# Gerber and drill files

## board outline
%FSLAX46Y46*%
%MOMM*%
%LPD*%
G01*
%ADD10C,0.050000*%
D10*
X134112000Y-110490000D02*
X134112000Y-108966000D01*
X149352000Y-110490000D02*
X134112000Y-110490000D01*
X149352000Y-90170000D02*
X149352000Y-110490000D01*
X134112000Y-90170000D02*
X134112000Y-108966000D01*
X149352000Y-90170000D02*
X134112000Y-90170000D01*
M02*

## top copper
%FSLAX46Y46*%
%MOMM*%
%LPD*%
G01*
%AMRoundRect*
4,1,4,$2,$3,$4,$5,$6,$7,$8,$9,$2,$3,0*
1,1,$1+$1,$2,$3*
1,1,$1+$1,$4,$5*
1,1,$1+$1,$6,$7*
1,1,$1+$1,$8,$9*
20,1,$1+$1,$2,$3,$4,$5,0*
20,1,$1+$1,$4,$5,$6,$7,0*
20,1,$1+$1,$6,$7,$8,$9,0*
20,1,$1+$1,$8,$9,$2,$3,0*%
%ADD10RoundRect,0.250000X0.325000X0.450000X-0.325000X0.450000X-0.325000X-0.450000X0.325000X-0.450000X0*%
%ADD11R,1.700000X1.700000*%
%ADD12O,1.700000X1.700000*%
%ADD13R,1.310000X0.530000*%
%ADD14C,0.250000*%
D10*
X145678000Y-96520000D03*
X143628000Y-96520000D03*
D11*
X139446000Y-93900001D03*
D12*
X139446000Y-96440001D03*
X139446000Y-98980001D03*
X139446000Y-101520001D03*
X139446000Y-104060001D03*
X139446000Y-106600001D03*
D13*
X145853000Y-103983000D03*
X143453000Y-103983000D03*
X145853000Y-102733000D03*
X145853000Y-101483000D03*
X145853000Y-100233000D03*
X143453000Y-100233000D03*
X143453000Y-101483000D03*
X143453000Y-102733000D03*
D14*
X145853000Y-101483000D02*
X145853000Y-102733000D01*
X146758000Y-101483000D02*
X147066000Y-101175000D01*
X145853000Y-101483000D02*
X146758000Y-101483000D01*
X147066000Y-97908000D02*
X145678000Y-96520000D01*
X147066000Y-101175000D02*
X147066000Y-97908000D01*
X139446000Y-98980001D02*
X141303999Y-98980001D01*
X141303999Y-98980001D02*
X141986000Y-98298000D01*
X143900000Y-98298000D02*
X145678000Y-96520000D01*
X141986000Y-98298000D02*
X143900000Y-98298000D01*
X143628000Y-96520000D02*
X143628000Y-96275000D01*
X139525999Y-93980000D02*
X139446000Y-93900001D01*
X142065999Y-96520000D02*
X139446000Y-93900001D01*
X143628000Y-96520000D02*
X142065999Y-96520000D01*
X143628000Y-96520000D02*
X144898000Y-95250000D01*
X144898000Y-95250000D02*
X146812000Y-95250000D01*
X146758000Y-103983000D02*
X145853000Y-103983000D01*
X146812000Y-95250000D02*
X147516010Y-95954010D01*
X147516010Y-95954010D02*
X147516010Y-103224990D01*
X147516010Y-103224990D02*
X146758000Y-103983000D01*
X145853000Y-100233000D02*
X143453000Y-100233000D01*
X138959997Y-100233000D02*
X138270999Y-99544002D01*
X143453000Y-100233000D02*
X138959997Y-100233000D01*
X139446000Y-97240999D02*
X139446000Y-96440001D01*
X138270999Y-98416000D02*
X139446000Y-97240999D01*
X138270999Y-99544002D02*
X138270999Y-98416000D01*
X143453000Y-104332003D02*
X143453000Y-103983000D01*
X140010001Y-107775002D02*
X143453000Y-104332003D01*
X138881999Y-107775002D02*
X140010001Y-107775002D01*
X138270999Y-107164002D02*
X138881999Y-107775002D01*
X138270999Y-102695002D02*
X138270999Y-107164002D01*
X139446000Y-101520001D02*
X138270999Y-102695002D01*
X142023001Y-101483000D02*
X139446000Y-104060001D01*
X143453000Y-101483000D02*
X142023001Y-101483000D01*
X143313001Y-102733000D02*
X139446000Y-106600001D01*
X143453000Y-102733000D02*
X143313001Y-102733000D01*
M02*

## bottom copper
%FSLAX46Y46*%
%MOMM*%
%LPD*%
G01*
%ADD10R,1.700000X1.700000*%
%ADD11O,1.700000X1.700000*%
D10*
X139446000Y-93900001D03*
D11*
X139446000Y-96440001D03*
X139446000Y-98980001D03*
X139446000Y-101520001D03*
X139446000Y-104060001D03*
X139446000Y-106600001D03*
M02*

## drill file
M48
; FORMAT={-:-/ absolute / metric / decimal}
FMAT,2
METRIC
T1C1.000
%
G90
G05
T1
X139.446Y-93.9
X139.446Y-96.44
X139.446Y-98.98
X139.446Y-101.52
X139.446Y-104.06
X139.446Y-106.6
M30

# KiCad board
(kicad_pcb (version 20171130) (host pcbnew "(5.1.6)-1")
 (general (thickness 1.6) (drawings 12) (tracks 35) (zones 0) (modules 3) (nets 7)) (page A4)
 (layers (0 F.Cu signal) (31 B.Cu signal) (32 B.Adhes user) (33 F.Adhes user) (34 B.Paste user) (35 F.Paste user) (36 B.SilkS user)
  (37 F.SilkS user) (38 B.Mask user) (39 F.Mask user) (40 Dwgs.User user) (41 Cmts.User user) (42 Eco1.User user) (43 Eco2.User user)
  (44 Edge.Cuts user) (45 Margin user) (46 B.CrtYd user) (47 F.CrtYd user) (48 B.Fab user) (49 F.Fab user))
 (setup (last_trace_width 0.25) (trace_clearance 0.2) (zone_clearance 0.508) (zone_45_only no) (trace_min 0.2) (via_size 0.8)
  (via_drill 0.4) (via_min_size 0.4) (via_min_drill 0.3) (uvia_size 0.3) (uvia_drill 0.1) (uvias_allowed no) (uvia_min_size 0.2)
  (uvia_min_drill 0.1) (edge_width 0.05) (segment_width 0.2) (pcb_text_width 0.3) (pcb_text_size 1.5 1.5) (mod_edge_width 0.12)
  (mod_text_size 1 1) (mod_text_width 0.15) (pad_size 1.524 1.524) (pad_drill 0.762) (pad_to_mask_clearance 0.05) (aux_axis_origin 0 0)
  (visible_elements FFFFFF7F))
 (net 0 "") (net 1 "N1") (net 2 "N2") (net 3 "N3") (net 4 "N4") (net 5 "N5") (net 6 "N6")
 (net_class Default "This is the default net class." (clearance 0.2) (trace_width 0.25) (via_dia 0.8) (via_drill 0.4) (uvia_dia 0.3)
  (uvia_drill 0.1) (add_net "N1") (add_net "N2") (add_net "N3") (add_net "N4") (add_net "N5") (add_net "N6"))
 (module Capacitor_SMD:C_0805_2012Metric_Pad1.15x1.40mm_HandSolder (layer F.Cu) (at 144.653 96.52 180)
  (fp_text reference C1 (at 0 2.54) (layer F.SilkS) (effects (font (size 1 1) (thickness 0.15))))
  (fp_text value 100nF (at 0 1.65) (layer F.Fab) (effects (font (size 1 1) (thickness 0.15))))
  (pad 1 smd roundrect (at -1.025 0 180) (size 1.15 1.4) (layers F.Cu F.Paste F.Mask) (roundrect_rratio 0.217391) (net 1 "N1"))
  (pad 2 smd roundrect (at 1.025 0 180) (size 1.15 1.4) (layers F.Cu F.Paste F.Mask) (roundrect_rratio 0.217391) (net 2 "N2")))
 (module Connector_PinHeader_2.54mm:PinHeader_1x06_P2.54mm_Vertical (layer F.Cu) (at 139.446 93.900001)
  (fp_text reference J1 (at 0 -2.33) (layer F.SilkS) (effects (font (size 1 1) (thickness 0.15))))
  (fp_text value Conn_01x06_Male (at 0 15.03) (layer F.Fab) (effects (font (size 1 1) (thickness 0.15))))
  (pad 1 thru_hole rect (at 0 0) (size 1.7 1.7) (drill 1) (layers *.Cu *.Mask) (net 2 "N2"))
  (pad 2 thru_hole oval (at 0 2.54) (size 1.7 1.7) (drill 1) (layers *.Cu *.Mask) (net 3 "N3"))
  (pad 3 thru_hole oval (at 0 5.08) (size 1.7 1.7) (drill 1) (layers *.Cu *.Mask) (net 1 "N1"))
  (pad 4 thru_hole oval (at 0 7.62) (size 1.7 1.7) (drill 1) (layers *.Cu *.Mask) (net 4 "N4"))
  (pad 5 thru_hole oval (at 0 10.16) (size 1.7 1.7) (drill 1) (layers *.Cu *.Mask) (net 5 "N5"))
  (pad 6 thru_hole oval (at 0 12.7) (size 1.7 1.7) (drill 1) (layers *.Cu *.Mask) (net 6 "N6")))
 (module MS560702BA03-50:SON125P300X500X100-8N (layer F.Cu) (at 144.653 102.108 180)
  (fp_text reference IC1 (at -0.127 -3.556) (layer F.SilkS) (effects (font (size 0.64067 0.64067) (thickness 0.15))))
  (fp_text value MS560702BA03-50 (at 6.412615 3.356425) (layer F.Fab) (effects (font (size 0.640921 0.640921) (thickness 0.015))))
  (pad 1 smd rect (at -1.2 -1.875 180) (size 1.31 0.53) (layers F.Cu F.Paste F.Mask) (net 2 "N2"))
  (pad 8 smd rect (at 1.2 -1.875 180) (size 1.31 0.53) (layers F.Cu F.Paste F.Mask) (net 4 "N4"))
  (pad 2 smd rect (at -1.2 -0.625 180) (size 1.31 0.53) (layers F.Cu F.Paste F.Mask) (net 1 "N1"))
  (pad 3 smd rect (at -1.2 0.625 180) (size 1.31 0.53) (layers F.Cu F.Paste F.Mask) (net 1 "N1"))
  (pad 4 smd rect (at -1.2 1.875 180) (size 1.31 0.53) (layers F.Cu F.Paste F.Mask) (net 3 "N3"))
  (pad 5 smd rect (at 1.2 1.875 180) (size 1.31 0.53) (layers F.Cu F.Paste F.Mask) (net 3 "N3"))
  (pad 6 smd rect (at 1.2 0.625 180) (size 1.31 0.53) (layers F.Cu F.Paste F.Mask) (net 5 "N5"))
  (pad 7 smd rect (at 1.2 -0.625 180) (size 1.31 0.53) (layers F.Cu F.Paste F.Mask) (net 6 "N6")))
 (gr_line (start 134.112 110.49) (end 134.112 108.966) (layer Edge.Cuts) (width 0.05))
 (gr_line (start 149.352 110.49) (end 134.112 110.49) (layer Edge.Cuts) (width 0.05))
 (gr_line (start 149.352 90.17) (end 149.352 110.49) (layer Edge.Cuts) (width 0.05))
 (gr_line (start 134.112 90.17) (end 134.112 108.966) (layer Edge.Cuts) (width 0.05))
 (gr_line (start 149.352 90.17) (end 134.112 90.17) (layer Edge.Cuts) (width 0.05))
 (segment (start 145.853 101.483) (end 145.853 102.733) (width 0.25) (layer F.Cu) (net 1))
 (segment (start 146.758 101.483) (end 147.066 101.175) (width 0.25) (layer F.Cu) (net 1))
 (segment (start 145.853 101.483) (end 146.758 101.483) (width 0.25) (layer F.Cu) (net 1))
 (segment (start 147.066 97.908) (end 145.678 96.52) (width 0.25) (layer F.Cu) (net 1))
 (segment (start 147.066 101.175) (end 147.066 97.908) (width 0.25) (layer F.Cu) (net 1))
 (segment (start 139.446 98.980001) (end 141.303999 98.980001) (width 0.25) (layer F.Cu) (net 1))
 (segment (start 141.303999 98.980001) (end 141.986 98.298) (width 0.25) (layer F.Cu) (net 1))
 (segment (start 143.9 98.298) (end 145.678 96.52) (width 0.25) (layer F.Cu) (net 1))
 (segment (start 141.986 98.298) (end 143.9 98.298) (width 0.25) (layer F.Cu) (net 1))
 (segment (start 143.628 96.52) (end 143.628 96.275) (width 0.25) (layer F.Cu) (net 2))
 (segment (start 139.525999 93.98) (end 139.446 93.900001) (width 0.25) (layer F.Cu) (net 2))
 (segment (start 142.065999 96.52) (end 139.446 93.900001) (width 0.25) (layer F.Cu) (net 2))
 (segment (start 143.628 96.52) (end 142.065999 96.52) (width 0.25) (layer F.Cu) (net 2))
 (segment (start 143.628 96.52) (end 144.898 95.25) (width 0.25) (layer F.Cu) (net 2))
 (segment (start 144.898 95.25) (end 146.812 95.25) (width 0.25) (layer F.Cu) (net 2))
 (segment (start 146.758 103.983) (end 145.853 103.983) (width 0.25) (layer F.Cu) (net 2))
 (segment (start 146.812 95.25) (end 147.51601 95.95401) (width 0.25) (layer F.Cu) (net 2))
 (segment (start 147.51601 95.95401) (end 147.51601 103.22499) (width 0.25) (layer F.Cu) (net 2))
 (segment (start 147.51601 103.22499) (end 146.758 103.983) (width 0.25) (layer F.Cu) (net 2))
 (segment (start 145.853 100.233) (end 143.453 100.233) (width 0.25) (layer F.Cu) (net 3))
 (segment (start 138.959997 100.233) (end 138.270999 99.544002) (width 0.25) (layer F.Cu) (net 3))
 (segment (start 143.453 100.233) (end 138.959997 100.233) (width 0.25) (layer F.Cu) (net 3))
 (segment (start 139.446 97.240999) (end 139.446 96.440001) (width 0.25) (layer F.Cu) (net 3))
 (segment (start 138.270999 98.416) (end 139.446 97.240999) (width 0.25) (layer F.Cu) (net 3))
 (segment (start 138.270999 99.544002) (end 138.270999 98.416) (width 0.25) (layer F.Cu) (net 3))
 (segment (start 143.453 104.332003) (end 143.453 103.983) (width 0.25) (layer F.Cu) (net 4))
 (segment (start 140.010001 107.775002) (end 143.453 104.332003) (width 0.25) (layer F.Cu) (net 4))
 (segment (start 138.881999 107.775002) (end 140.010001 107.775002) (width 0.25) (layer F.Cu) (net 4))
 (segment (start 138.270999 107.164002) (end 138.881999 107.775002) (width 0.25) (layer F.Cu) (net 4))
 (segment (start 138.270999 102.695002) (end 138.270999 107.164002) (width 0.25) (layer F.Cu) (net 4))
 (segment (start 139.446 101.520001) (end 138.270999 102.695002) (width 0.25) (layer F.Cu) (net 4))
 (segment (start 142.023001 101.483) (end 139.446 104.060001) (width 0.25) (layer F.Cu) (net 5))
 (segment (start 143.453 101.483) (end 142.023001 101.483) (width 0.25) (layer F.Cu) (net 5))
 (segment (start 143.313001 102.733) (end 139.446 106.600001) (width 0.25) (layer F.Cu) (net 6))
 (segment (start 143.453 102.733) (end 143.313001 102.733) (width 0.25) (layer F.Cu) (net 6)))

